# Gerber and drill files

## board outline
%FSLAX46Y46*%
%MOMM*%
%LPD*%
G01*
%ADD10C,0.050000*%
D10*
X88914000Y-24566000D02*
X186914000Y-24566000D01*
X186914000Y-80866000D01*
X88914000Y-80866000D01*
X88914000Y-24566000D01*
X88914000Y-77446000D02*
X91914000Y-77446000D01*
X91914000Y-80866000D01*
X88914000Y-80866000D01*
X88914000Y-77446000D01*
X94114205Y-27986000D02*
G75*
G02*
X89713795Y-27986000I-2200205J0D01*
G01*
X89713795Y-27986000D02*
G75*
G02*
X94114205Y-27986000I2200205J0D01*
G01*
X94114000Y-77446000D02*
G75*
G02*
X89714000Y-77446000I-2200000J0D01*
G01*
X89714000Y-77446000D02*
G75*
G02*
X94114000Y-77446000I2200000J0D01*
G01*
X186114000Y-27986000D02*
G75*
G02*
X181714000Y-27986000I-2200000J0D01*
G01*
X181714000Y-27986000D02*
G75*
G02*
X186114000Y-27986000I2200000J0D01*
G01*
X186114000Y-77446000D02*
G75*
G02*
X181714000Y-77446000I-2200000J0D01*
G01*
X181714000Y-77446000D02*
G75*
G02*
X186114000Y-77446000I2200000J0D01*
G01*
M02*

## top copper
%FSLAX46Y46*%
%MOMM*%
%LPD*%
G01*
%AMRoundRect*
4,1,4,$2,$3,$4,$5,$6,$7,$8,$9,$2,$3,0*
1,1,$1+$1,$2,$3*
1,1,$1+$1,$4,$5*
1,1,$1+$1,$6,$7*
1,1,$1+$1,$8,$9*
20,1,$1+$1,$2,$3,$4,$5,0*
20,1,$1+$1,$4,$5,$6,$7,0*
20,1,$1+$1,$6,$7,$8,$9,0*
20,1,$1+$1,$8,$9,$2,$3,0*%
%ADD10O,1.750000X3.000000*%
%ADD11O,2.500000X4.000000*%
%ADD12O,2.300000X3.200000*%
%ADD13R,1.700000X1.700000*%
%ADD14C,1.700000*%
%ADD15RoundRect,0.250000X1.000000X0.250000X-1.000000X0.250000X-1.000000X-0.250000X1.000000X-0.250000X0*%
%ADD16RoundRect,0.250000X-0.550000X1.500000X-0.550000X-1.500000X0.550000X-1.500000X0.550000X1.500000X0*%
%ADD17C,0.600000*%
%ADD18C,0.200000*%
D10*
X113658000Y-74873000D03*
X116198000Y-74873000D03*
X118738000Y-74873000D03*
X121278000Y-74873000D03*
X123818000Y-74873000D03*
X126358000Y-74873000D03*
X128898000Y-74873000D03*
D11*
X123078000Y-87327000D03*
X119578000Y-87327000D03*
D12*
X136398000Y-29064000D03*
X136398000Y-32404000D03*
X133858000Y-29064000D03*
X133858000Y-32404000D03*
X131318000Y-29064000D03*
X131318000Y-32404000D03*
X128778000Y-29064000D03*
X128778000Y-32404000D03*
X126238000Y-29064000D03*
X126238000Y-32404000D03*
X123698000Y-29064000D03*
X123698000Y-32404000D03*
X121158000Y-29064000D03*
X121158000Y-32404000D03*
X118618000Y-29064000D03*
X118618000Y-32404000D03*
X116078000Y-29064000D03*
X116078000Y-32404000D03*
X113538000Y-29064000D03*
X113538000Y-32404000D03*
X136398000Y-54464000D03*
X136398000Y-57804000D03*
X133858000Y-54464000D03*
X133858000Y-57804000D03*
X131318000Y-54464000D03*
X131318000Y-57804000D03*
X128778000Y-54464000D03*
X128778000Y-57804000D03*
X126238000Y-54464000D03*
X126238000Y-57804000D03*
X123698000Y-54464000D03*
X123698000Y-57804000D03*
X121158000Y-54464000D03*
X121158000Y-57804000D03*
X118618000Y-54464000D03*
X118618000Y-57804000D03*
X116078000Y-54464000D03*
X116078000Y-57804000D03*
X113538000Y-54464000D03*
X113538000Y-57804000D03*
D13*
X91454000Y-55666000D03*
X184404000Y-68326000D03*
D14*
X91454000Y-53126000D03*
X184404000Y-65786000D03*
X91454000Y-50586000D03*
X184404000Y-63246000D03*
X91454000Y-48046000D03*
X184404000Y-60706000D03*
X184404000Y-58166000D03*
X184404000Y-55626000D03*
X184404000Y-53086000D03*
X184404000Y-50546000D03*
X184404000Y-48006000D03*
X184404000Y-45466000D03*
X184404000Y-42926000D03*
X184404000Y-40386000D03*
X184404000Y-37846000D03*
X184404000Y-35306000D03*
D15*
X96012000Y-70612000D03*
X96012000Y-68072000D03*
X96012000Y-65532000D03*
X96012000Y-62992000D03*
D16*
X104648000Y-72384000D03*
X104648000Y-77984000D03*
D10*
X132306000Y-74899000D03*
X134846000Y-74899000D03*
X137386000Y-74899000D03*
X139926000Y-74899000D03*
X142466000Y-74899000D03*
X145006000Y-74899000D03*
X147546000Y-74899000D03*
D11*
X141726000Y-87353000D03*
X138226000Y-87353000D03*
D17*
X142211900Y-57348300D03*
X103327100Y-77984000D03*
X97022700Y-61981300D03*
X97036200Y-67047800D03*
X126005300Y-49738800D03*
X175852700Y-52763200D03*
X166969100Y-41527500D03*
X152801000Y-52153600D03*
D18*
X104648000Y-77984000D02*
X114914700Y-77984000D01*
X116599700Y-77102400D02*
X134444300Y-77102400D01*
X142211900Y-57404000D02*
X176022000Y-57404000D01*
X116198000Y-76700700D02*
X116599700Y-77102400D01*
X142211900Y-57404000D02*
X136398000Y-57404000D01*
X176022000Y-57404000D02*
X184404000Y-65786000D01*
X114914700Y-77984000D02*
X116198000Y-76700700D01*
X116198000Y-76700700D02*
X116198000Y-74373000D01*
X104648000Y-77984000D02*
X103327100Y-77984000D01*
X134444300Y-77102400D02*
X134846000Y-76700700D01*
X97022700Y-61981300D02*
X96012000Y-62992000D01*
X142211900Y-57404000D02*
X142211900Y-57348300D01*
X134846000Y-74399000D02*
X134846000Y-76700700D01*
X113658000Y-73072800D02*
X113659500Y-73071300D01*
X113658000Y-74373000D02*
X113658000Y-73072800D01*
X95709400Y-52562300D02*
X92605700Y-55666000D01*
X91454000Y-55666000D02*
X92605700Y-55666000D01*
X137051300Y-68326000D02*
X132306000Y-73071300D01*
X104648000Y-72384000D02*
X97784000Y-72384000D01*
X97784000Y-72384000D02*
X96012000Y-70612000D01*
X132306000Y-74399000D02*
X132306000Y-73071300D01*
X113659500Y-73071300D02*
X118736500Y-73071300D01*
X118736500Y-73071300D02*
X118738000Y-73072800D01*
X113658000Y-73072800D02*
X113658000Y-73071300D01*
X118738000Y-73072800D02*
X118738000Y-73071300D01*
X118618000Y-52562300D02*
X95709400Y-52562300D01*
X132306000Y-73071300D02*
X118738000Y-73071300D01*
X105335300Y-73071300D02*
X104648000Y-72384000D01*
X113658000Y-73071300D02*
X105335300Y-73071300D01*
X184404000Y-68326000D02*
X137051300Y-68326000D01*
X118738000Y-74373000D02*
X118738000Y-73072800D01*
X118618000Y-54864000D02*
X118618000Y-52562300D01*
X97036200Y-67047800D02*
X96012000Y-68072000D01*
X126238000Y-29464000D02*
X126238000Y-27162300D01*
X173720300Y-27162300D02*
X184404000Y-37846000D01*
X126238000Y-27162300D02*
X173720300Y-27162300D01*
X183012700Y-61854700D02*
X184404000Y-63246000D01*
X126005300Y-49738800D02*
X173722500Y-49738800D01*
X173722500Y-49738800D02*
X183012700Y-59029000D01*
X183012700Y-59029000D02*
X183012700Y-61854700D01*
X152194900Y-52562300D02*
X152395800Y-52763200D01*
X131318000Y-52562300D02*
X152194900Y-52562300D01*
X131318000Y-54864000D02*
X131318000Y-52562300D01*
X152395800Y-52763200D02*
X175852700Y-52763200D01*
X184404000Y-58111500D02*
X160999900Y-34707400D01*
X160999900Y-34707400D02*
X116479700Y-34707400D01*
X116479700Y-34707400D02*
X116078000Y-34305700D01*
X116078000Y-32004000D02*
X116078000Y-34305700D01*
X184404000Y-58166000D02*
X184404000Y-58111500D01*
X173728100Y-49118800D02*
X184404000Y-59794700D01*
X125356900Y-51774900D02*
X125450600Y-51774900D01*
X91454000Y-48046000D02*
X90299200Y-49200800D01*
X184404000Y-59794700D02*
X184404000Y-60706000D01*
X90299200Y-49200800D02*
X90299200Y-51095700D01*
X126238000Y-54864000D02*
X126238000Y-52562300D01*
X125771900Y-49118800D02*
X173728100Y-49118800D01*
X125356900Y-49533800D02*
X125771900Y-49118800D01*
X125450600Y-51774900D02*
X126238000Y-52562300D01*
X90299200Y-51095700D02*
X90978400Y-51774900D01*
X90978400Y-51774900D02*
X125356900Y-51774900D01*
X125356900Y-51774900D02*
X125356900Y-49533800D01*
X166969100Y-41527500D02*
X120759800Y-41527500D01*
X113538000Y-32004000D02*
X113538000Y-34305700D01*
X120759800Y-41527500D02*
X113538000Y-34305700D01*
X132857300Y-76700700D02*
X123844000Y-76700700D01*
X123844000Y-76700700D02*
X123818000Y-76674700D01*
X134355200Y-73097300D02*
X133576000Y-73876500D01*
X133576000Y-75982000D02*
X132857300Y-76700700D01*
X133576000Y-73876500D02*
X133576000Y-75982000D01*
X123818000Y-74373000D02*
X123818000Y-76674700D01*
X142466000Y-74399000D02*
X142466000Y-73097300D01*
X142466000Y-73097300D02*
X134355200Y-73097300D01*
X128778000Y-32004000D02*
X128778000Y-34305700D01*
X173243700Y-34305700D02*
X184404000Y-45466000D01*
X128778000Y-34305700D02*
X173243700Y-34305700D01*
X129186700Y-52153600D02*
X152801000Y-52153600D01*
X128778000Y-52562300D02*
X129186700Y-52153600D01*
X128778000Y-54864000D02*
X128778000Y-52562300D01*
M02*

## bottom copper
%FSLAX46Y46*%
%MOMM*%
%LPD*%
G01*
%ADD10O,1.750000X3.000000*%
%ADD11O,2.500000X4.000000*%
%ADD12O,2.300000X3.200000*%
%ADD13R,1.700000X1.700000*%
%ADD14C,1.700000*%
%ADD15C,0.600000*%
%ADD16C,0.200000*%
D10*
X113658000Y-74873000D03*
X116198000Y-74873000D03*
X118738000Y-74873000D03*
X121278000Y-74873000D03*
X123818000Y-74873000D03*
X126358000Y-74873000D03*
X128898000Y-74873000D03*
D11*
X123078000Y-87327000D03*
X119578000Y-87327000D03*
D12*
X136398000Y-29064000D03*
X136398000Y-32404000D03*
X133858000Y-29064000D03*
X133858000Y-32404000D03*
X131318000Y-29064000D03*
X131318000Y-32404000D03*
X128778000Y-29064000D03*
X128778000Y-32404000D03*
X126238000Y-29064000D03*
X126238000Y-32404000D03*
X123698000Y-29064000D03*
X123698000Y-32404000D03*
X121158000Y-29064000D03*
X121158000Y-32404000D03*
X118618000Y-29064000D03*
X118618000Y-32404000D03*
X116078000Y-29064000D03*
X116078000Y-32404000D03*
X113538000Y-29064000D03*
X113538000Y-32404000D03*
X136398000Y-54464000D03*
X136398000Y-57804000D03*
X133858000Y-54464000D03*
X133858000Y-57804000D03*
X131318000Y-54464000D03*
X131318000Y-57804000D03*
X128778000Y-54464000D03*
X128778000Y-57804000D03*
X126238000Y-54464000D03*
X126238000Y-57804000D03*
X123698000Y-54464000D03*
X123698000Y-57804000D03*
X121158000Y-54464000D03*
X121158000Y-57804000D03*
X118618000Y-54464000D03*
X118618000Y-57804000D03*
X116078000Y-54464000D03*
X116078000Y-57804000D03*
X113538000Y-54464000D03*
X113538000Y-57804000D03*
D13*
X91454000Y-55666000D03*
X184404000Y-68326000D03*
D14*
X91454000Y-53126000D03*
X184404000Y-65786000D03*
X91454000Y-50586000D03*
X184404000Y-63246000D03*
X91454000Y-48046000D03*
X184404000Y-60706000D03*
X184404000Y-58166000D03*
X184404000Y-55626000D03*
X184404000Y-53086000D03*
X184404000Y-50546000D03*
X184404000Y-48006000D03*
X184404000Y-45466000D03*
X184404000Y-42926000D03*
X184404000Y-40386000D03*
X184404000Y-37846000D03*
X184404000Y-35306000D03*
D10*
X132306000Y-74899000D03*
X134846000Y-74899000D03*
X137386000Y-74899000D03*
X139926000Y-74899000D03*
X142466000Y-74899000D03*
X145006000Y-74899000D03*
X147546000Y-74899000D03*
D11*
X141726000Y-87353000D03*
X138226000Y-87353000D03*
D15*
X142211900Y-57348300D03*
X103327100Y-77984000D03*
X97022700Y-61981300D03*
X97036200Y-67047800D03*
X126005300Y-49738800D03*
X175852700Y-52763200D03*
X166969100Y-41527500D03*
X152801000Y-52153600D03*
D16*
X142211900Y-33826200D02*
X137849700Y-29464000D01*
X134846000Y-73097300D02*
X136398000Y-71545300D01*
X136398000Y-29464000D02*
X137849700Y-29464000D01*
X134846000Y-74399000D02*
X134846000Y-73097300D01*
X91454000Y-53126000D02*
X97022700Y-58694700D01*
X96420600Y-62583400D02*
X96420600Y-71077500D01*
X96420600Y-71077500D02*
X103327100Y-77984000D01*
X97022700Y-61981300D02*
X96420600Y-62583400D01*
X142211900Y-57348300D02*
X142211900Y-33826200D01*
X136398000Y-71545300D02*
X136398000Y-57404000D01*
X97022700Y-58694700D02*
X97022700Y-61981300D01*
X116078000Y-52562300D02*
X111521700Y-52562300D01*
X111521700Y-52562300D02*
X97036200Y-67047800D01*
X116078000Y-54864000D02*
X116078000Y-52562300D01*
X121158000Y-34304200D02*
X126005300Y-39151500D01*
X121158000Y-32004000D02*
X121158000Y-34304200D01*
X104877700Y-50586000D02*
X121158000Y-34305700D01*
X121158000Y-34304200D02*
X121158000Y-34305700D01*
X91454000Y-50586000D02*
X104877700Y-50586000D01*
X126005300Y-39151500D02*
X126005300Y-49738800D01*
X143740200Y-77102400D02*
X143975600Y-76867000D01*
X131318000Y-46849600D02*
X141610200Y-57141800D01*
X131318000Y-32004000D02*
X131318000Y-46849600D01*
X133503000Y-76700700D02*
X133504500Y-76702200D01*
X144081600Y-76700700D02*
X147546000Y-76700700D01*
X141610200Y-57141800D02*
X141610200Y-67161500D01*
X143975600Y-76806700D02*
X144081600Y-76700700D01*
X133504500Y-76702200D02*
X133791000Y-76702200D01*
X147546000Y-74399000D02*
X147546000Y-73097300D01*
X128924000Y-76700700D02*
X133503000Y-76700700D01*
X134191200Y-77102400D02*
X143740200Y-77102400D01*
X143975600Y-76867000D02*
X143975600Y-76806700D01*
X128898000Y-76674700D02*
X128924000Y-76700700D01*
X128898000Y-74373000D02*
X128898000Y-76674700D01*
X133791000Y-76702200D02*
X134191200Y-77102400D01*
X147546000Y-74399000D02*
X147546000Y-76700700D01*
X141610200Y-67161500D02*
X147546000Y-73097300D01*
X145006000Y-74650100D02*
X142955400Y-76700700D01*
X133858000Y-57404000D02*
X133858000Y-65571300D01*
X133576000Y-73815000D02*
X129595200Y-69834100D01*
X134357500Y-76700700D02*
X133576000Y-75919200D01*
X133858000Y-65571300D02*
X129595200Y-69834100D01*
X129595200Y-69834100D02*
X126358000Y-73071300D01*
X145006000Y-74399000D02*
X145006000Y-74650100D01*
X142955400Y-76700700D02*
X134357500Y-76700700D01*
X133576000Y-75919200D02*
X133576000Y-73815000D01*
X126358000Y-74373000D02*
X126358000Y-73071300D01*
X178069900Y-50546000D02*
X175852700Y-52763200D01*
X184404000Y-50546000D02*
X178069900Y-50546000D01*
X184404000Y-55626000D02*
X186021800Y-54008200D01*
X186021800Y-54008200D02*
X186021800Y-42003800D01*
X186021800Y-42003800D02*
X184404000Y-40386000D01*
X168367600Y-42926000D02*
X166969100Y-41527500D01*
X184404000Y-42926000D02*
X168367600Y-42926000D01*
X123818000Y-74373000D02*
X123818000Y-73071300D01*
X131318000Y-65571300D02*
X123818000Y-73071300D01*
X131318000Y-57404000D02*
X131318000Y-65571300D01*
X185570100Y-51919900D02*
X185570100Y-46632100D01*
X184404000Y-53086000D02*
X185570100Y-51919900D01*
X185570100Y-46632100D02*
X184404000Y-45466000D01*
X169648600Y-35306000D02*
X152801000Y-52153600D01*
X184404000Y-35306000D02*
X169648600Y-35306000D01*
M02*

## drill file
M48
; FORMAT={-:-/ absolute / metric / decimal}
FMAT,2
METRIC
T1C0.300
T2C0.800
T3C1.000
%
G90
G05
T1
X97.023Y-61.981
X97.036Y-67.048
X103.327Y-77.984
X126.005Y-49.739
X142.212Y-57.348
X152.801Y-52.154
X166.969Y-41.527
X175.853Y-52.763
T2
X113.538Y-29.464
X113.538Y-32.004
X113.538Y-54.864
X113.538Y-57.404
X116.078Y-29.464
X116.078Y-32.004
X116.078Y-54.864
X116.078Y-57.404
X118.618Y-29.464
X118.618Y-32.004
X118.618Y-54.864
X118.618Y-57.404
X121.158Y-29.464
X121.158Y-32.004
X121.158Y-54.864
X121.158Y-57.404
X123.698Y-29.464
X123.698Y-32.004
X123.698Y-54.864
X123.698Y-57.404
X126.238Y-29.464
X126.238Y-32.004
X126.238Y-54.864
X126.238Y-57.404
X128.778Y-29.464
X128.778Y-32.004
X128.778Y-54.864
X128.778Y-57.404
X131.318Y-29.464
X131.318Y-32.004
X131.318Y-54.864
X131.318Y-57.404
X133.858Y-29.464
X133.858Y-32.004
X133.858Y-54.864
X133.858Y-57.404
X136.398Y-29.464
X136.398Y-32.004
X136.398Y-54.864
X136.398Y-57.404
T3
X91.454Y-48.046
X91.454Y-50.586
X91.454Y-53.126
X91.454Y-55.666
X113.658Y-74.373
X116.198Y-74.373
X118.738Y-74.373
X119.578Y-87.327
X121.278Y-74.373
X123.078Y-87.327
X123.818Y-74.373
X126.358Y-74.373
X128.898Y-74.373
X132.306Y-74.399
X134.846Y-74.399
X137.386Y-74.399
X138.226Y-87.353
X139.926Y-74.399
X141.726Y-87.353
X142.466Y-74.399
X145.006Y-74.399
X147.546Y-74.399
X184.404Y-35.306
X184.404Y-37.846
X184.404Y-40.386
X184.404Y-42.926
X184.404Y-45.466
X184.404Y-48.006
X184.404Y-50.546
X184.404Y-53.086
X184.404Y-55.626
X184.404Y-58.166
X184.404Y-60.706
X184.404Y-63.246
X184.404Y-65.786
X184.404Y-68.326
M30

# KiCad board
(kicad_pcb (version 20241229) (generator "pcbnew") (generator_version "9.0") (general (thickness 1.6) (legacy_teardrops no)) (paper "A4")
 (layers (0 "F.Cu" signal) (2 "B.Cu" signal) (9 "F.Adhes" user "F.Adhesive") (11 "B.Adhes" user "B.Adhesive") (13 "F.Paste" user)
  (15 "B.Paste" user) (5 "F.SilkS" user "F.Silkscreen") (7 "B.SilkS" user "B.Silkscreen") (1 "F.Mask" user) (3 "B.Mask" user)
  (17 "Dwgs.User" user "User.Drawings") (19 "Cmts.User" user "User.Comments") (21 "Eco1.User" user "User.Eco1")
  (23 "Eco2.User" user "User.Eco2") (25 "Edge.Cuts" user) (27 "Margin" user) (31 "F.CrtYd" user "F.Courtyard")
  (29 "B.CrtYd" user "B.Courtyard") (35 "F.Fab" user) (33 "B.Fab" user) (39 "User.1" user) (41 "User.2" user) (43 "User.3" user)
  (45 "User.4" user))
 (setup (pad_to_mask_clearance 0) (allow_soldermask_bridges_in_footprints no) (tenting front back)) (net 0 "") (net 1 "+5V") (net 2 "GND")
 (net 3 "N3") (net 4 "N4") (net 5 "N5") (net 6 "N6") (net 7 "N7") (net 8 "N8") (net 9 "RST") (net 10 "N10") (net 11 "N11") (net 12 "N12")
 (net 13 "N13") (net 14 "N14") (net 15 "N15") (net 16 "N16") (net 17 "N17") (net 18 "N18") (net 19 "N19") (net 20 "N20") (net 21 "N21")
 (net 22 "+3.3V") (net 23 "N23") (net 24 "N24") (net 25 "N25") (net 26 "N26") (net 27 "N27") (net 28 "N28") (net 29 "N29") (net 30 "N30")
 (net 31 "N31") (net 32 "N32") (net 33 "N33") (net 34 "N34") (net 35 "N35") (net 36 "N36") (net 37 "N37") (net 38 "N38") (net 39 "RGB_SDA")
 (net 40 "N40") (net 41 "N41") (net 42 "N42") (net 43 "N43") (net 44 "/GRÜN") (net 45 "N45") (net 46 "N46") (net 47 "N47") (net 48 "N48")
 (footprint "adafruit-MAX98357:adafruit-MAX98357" (layer "F.Cu") (at 121.158 81.28 180)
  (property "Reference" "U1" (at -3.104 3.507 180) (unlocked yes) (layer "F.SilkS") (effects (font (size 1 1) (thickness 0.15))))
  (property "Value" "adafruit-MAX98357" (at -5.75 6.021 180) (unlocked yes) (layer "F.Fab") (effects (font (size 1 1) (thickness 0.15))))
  (pad "1" thru_hole oval (at 7.5 6.907 90) (size 3 1.75) (drill 1 (offset -0.5 0)) (layers "*.Cu" "*.Mask") (remove_unused_layers no)
   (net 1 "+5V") (solder_mask_margin 0.0508))
  (pad "2" thru_hole oval (at 4.96 6.907 90) (size 3 1.75) (drill 1 (offset -0.5 0)) (layers "*.Cu" "*.Mask") (remove_unused_layers no)
   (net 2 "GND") (solder_mask_margin 0.0508))
  (pad "3" thru_hole oval (at 2.42 6.907 90) (size 3 1.75) (drill 1 (offset -0.5 0)) (layers "*.Cu" "*.Mask") (remove_unused_layers no)
   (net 1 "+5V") (solder_mask_margin 0.0508))
  (pad "4" thru_hole oval (at -0.12 6.907 90) (size 3 1.75) (drill 1 (offset -0.5 0)) (layers "*.Cu" "*.Mask") (remove_unused_layers no)
   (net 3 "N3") (solder_mask_margin 0.0508))
  (pad "5" thru_hole oval (at -2.66 6.907 90) (size 3 1.75) (drill 1 (offset -0.5 0)) (layers "*.Cu" "*.Mask") (remove_unused_layers no)
   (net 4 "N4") (solder_mask_margin 0.0508))
  (pad "6" thru_hole oval (at -5.2 6.907 90) (size 3 1.75) (drill 1 (offset -0.5 0)) (layers "*.Cu" "*.Mask") (remove_unused_layers no)
   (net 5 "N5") (solder_mask_margin 0.0508))
  (pad "7" thru_hole oval (at -7.74 6.907 90) (size 3 1.75) (drill 1 (offset -0.5 0)) (layers "*.Cu" "*.Mask") (remove_unused_layers no)
   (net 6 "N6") (solder_mask_margin 0.0508))
  (pad "8" thru_hole oval (at -1.92 -6.047) (size 2.5 4) (drill 1) (layers "*.Cu" "*.Mask") (remove_unused_layers no) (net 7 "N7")
   (solder_mask_margin 0.0508))
  (pad "9" thru_hole oval (at 1.58 -6.047) (size 2.5 4) (drill 1) (layers "*.Cu" "*.Mask") (remove_unused_layers no) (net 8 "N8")
   (solder_mask_margin 0.0508)))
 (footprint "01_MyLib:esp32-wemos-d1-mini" (layer "F.Cu") (at 124.968 43.434 -90)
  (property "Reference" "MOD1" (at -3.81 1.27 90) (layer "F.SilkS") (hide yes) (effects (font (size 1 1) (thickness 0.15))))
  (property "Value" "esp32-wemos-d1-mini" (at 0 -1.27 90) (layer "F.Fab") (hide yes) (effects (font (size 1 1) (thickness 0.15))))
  (pad "1" thru_hole oval (at -13.97 -11.43 180) (size 2.3 3.2) (drill 0.8 (offset 0 0.4)) (layers "*.Cu" "*.Mask")
   (remove_unused_layers no) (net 2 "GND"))
  (pad "2" thru_hole oval (at -11.43 -11.43 180) (size 2.3 3.2) (drill 0.8 (offset 0 -0.4)) (layers "*.Cu" "*.Mask")
   (remove_unused_layers no) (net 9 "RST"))
  (pad "3" thru_hole oval (at -13.97 -8.89 180) (size 2.3 3.2) (drill 0.8 (offset 0 0.4)) (layers "*.Cu" "*.Mask") (remove_unused_layers no)
   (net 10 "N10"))
  (pad "4" thru_hole oval (at -11.43 -8.89 180) (size 2.3 3.2) (drill 0.8 (offset 0 -0.4)) (layers "*.Cu" "*.Mask")
   (remove_unused_layers no) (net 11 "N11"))
  (pad "5" thru_hole oval (at -13.97 -6.35 180) (size 2.3 3.2) (drill 0.8 (offset 0 0.4)) (layers "*.Cu" "*.Mask") (remove_unused_layers no)
   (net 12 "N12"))
  (pad "6" thru_hole oval (at -11.43 -6.35 180) (size 2.3 3.2) (drill 0.8 (offset 0 -0.4)) (layers "*.Cu" "*.Mask")
   (remove_unused_layers no) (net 6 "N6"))
  (pad "7" thru_hole oval (at -13.97 -3.81 180) (size 2.3 3.2) (drill 0.8 (offset 0 0.4)) (layers "*.Cu" "*.Mask") (remove_unused_layers no)
   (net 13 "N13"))
  (pad "8" thru_hole oval (at -11.43 -3.81 180) (size 2.3 3.2) (drill 0.8 (offset 0 -0.4)) (layers "*.Cu" "*.Mask")
   (remove_unused_layers no) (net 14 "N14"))
  (pad "9" thru_hole oval (at -13.97 -1.27 180) (size 2.3 3.2) (drill 0.8 (offset 0 0.4)) (layers "*.Cu" "*.Mask") (remove_unused_layers no)
   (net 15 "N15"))
  (pad "10" thru_hole oval (at -11.43 -1.27 180) (size 2.3 3.2) (drill 0.8 (offset 0 -0.4)) (layers "*.Cu" "*.Mask")
   (remove_unused_layers no) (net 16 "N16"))
  (pad "11" thru_hole oval (at -13.97 1.27 180) (size 2.3 3.2) (drill 0.8 (offset 0 0.4)) (layers "*.Cu" "*.Mask") (remove_unused_layers no)
   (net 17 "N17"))
  (pad "12" thru_hole oval (at -11.43 1.27 180) (size 2.3 3.2) (drill 0.8 (offset 0 -0.4)) (layers "*.Cu" "*.Mask")
   (remove_unused_layers no) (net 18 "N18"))
  (pad "13" thru_hole oval (at -13.97 3.81 180) (size 2.3 3.2) (drill 0.8 (offset 0 0.4)) (layers "*.Cu" "*.Mask") (remove_unused_layers no)
   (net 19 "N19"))
  (pad "14" thru_hole oval (at -11.43 3.81 180) (size 2.3 3.2) (drill 0.8 (offset 0 -0.4)) (layers "*.Cu" "*.Mask")
   (remove_unused_layers no) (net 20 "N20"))
  (pad "15" thru_hole oval (at -13.97 6.35 180) (size 2.3 3.2) (drill 0.8 (offset 0 0.4)) (layers "*.Cu" "*.Mask") (remove_unused_layers no)
   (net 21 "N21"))
  (pad "16" thru_hole oval (at -11.43 6.35 180) (size 2.3 3.2) (drill 0.8 (offset 0 -0.4)) (layers "*.Cu" "*.Mask")
   (remove_unused_layers no) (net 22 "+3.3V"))
  (pad "17" thru_hole oval (at -13.97 8.89 180) (size 2.3 3.2) (drill 0.8 (offset 0 0.4)) (layers "*.Cu" "*.Mask") (remove_unused_layers no)
   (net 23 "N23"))
  (pad "18" thru_hole oval (at -11.43 8.89 180) (size 2.3 3.2) (drill 0.8 (offset 0 -0.4)) (layers "*.Cu" "*.Mask")
   (remove_unused_layers no) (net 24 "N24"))
  (pad "19" thru_hole oval (at -13.97 11.43 180) (size 2.3 3.2) (drill 0.8 (offset 0 0.4)) (layers "*.Cu" "*.Mask")
   (remove_unused_layers no) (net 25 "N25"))
  (pad "20" thru_hole oval (at -11.43 11.43 180) (size 2.3 3.2) (drill 0.8 (offset 0 -0.4)) (layers "*.Cu" "*.Mask")
   (remove_unused_layers no) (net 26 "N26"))
  (pad "21" thru_hole oval (at 11.43 -11.43 180) (size 2.3 3.2) (drill 0.8 (offset 0 0.4)) (layers "*.Cu" "*.Mask")
   (remove_unused_layers no) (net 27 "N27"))
  (pad "22" thru_hole oval (at 13.97 -11.43 180) (size 2.3 3.2) (drill 0.8 (offset 0 -0.4)) (layers "*.Cu" "*.Mask")
   (remove_unused_layers no) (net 2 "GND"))
  (pad "23" thru_hole oval (at 11.43 -8.89 180) (size 2.3 3.2) (drill 0.8 (offset 0 0.4)) (layers "*.Cu" "*.Mask") (remove_unused_layers no)
   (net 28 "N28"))
  (pad "24" thru_hole oval (at 13.97 -8.89 180) (size 2.3 3.2) (drill 0.8 (offset 0 -0.4)) (layers "*.Cu" "*.Mask")
   (remove_unused_layers no) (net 5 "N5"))
  (pad "25" thru_hole oval (at 11.43 -6.35 180) (size 2.3 3.2) (drill 0.8 (offset 0 0.4)) (layers "*.Cu" "*.Mask") (remove_unused_layers no)
   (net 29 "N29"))
  (pad "26" thru_hole oval (at 13.97 -6.35 180) (size 2.3 3.2) (drill 0.8 (offset 0 -0.4)) (layers "*.Cu" "*.Mask")
   (remove_unused_layers no) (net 4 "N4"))
  (pad "27" thru_hole oval (at 11.43 -3.81 180) (size 2.3 3.2) (drill 0.8 (offset 0 0.4)) (layers "*.Cu" "*.Mask") (remove_unused_layers no)
   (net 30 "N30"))
  (pad "28" thru_hole oval (at 13.97 -3.81 180) (size 2.3 3.2) (drill 0.8 (offset 0 -0.4)) (layers "*.Cu" "*.Mask")
   (remove_unused_layers no) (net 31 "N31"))
  (pad "29" thru_hole oval (at 11.43 -1.27 180) (size 2.3 3.2) (drill 0.8 (offset 0 0.4)) (layers "*.Cu" "*.Mask") (remove_unused_layers no)
   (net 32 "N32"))
  (pad "30" thru_hole oval (at 13.97 -1.27 180) (size 2.3 3.2) (drill 0.8 (offset 0 -0.4)) (layers "*.Cu" "*.Mask")
   (remove_unused_layers no) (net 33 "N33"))
  (pad "31" thru_hole oval (at 11.43 1.27 180) (size 2.3 3.2) (drill 0.8 (offset 0 0.4)) (layers "*.Cu" "*.Mask") (remove_unused_layers no)
   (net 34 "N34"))
  (pad "32" thru_hole oval (at 13.97 1.27 180) (size 2.3 3.2) (drill 0.8 (offset 0 -0.4)) (layers "*.Cu" "*.Mask") (remove_unused_layers no)
   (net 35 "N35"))
  (pad "33" thru_hole oval (at 11.43 3.81 180) (size 2.3 3.2) (drill 0.8 (offset 0 0.4)) (layers "*.Cu" "*.Mask") (remove_unused_layers no)
   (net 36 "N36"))
  (pad "34" thru_hole oval (at 13.97 3.81 180) (size 2.3 3.2) (drill 0.8 (offset 0 -0.4)) (layers "*.Cu" "*.Mask") (remove_unused_layers no)
   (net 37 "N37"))
  (pad "35" thru_hole oval (at 11.43 6.35 180) (size 2.3 3.2) (drill 0.8 (offset 0 0.4)) (layers "*.Cu" "*.Mask") (remove_unused_layers no)
   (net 1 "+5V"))
  (pad "36" thru_hole oval (at 13.97 6.35 180) (size 2.3 3.2) (drill 0.8 (offset 0 -0.4)) (layers "*.Cu" "*.Mask") (remove_unused_layers no)
   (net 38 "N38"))
  (pad "37" thru_hole oval (at 11.43 8.89 180) (size 2.3 3.2) (drill 0.8 (offset 0 0.4)) (layers "*.Cu" "*.Mask") (remove_unused_layers no)
   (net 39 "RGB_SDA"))
  (pad "38" thru_hole oval (at 13.97 8.89 180) (size 2.3 3.2) (drill 0.8 (offset 0 -0.4)) (layers "*.Cu" "*.Mask") (remove_unused_layers no)
   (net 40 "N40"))
  (pad "39" thru_hole oval (at 11.43 11.43 180) (size 2.3 3.2) (drill 0.8 (offset 0 0.4)) (layers "*.Cu" "*.Mask") (remove_unused_layers no)
   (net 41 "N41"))
  (pad "40" thru_hole oval (at 13.97 11.43 180) (size 2.3 3.2) (drill 0.8 (offset 0 -0.4)) (layers "*.Cu" "*.Mask")
   (remove_unused_layers no) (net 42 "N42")))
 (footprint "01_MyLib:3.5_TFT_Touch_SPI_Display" (layer "F.Cu") (at 88.914 80.866)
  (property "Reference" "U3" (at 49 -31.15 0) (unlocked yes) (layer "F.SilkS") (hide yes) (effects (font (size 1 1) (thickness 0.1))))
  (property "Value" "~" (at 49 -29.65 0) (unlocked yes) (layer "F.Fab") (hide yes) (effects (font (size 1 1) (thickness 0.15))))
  (fp_rect (start 0 -56.3) (end 98 0) (stroke (width 0.05) (type default)) (fill no) (layer "Edge.Cuts"))
  (fp_rect (start 0 -3.42) (end 3 0) (stroke (width 0.05) (type default)) (fill no) (layer "Edge.Cuts"))
  (fp_circle (center 3 -52.88) (end 5.2 -52.91) (stroke (width 0.05) (type default)) (fill no) (layer "Edge.Cuts"))
  (fp_circle (center 3 -3.42) (end 5.2 -3.42) (stroke (width 0.05) (type default)) (fill no) (layer "Edge.Cuts"))
  (fp_circle (center 95 -52.88) (end 92.8 -52.88) (stroke (width 0.05) (type default)) (fill no) (layer "Edge.Cuts"))
  (fp_circle (center 95 -3.42) (end 92.8 -3.42) (stroke (width 0.05) (type default)) (fill no) (layer "Edge.Cuts"))
  (pad "1" thru_hole rect (at 2.54 -25.2 180) (size 1.7 1.7) (drill 1) (layers "*.Cu" "*.Mask") (remove_unused_layers no) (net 1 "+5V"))
  (pad "1" thru_hole rect (at 95.49 -12.54 180) (size 1.7 1.7) (drill 1) (layers "*.Cu" "*.Mask") (remove_unused_layers no) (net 1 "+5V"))
  (pad "2" thru_hole circle (at 2.54 -27.74 180) (size 1.7 1.7) (drill 1) (layers "*.Cu" "*.Mask") (remove_unused_layers no) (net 2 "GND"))
  (pad "2" thru_hole circle (at 95.49 -15.08 180) (size 1.7 1.7) (drill 1) (layers "*.Cu" "*.Mask") (remove_unused_layers no) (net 2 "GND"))
  (pad "3" thru_hole circle (at 2.54 -30.28 180) (size 1.7 1.7) (drill 1) (layers "*.Cu" "*.Mask") (remove_unused_layers no) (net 20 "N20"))
  (pad "3" thru_hole circle (at 95.49 -17.62 180) (size 1.7 1.7) (drill 1) (layers "*.Cu" "*.Mask") (remove_unused_layers no) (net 20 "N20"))
  (pad "4" thru_hole circle (at 2.54 -32.82 180) (size 1.7 1.7) (drill 1) (layers "*.Cu" "*.Mask") (remove_unused_layers no) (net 32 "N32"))
  (pad "4" thru_hole circle (at 95.49 -20.16 180) (size 1.7 1.7) (drill 1) (layers "*.Cu" "*.Mask") (remove_unused_layers no) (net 32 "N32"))
  (pad "5" thru_hole circle (at 95.49 -22.7 180) (size 1.7 1.7) (drill 1) (layers "*.Cu" "*.Mask") (remove_unused_layers no) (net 24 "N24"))
  (pad "6" thru_hole circle (at 95.49 -25.24 180) (size 1.7 1.7) (drill 1) (layers "*.Cu" "*.Mask") (remove_unused_layers no) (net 17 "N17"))
  (pad "7" thru_hole circle (at 95.49 -27.78 180) (size 1.7 1.7) (drill 1) (layers "*.Cu" "*.Mask") (remove_unused_layers no) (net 14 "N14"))
  (pad "8" thru_hole circle (at 95.49 -30.32 180) (size 1.7 1.7) (drill 1) (layers "*.Cu" "*.Mask") (remove_unused_layers no) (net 29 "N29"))
  (pad "9" thru_hole circle (at 95.49 -32.86 180) (size 1.7 1.7) (drill 1) (layers "*.Cu" "*.Mask") (remove_unused_layers no) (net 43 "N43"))
  (pad "10" thru_hole circle (at 95.49 -35.4 180) (size 1.7 1.7) (drill 1) (layers "*.Cu" "*.Mask") (remove_unused_layers no) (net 14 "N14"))
  (pad "11" thru_hole circle (at 95.49 -37.94 180) (size 1.7 1.7) (drill 1) (layers "*.Cu" "*.Mask") (remove_unused_layers no)
   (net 26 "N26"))
  (pad "12" thru_hole circle (at 95.49 -40.48 180) (size 1.7 1.7) (drill 1) (layers "*.Cu" "*.Mask") (remove_unused_layers no)
   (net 17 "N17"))
  (pad "13" thru_hole circle (at 95.49 -43.02 180) (size 1.7 1.7) (drill 1) (layers "*.Cu" "*.Mask") (remove_unused_layers no)
   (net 15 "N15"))
  (pad "14" thru_hole circle (at 95.49 -45.56 180) (size 1.7 1.7) (drill 1) (layers "*.Cu" "*.Mask") (remove_unused_layers no)
   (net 30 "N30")))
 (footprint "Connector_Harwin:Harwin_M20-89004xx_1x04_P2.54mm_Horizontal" (layer "F.Cu") (at 90.487 66.802 180)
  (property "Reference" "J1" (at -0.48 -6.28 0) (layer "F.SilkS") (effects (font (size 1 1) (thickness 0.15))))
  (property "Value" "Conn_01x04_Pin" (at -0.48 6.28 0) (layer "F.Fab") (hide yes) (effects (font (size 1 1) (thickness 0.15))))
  (pad "1" smd roundrect (at -5.525 -3.81 180) (size 2.5 1) (layers "F.Cu" "F.Mask" "F.Paste") (roundrect_rratio 0.25) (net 1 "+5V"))
  (pad "2" smd roundrect (at -5.525 -1.27 180) (size 2.5 1) (layers "F.Cu" "F.Mask" "F.Paste") (roundrect_rratio 0.25) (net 39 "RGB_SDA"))
  (pad "3" smd roundrect (at -5.525 1.27 180) (size 2.5 1) (layers "F.Cu" "F.Mask" "F.Paste") (roundrect_rratio 0.25) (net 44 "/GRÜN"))
  (pad "4" smd roundrect (at -5.525 3.81 180) (size 2.5 1) (layers "F.Cu" "F.Mask" "F.Paste") (roundrect_rratio 0.25) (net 2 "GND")))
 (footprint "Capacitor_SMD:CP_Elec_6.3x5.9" (layer "F.Cu") (at 104.648 75.184 -90)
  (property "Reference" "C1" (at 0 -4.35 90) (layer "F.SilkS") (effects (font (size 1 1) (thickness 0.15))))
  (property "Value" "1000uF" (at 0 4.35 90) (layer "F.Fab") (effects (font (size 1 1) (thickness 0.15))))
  (pad "1" smd roundrect (at -2.8 0 270) (size 3.5 1.6) (layers "F.Cu" "F.Mask" "F.Paste") (roundrect_rratio 0.15625) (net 1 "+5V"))
  (pad "2" smd roundrect (at 2.8 0 270) (size 3.5 1.6) (layers "F.Cu" "F.Mask" "F.Paste") (roundrect_rratio 0.15625) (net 2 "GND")))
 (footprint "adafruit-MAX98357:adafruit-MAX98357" (layer "F.Cu") (at 139.806 81.306 180)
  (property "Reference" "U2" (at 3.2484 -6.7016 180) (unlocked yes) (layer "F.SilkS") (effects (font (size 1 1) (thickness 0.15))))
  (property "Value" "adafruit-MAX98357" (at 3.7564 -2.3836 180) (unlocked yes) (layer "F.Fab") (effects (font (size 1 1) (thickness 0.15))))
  (pad "1" thru_hole oval (at 7.5 6.907 90) (size 3 1.75) (drill 1 (offset -0.5 0)) (layers "*.Cu" "*.Mask") (remove_unused_layers no)
   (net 1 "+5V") (solder_mask_margin 0.0508))
  (pad "2" thru_hole oval (at 4.96 6.907 90) (size 3 1.75) (drill 1 (offset -0.5 0)) (layers "*.Cu" "*.Mask") (remove_unused_layers no)
   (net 2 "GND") (solder_mask_margin 0.0508))
  (pad "3" thru_hole oval (at 2.42 6.907 90) (size 3 1.75) (drill 1 (offset -0.5 0)) (layers "*.Cu" "*.Mask") (remove_unused_layers no)
   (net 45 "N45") (solder_mask_margin 0.0508))
  (pad "4" thru_hole oval (at -0.12 6.907 90) (size 3 1.75) (drill 1 (offset -0.5 0)) (layers "*.Cu" "*.Mask") (remove_unused_layers no)
   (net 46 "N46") (solder_mask_margin 0.0508))
  (pad "5" thru_hole oval (at -2.66 6.907 90) (size 3 1.75) (drill 1 (offset -0.5 0)) (layers "*.Cu" "*.Mask") (remove_unused_layers no)
   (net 4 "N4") (solder_mask_margin 0.0508))
  (pad "6" thru_hole oval (at -5.2 6.907 90) (size 3 1.75) (drill 1 (offset -0.5 0)) (layers "*.Cu" "*.Mask") (remove_unused_layers no)
   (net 5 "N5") (solder_mask_margin 0.0508))
  (pad "7" thru_hole oval (at -7.74 6.907 90) (size 3 1.75) (drill 1 (offset -0.5 0)) (layers "*.Cu" "*.Mask") (remove_unused_layers no)
   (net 6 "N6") (solder_mask_margin 0.0508))
  (pad "8" thru_hole oval (at -1.92 -6.047) (size 2.5 4) (drill 1) (layers "*.Cu" "*.Mask") (remove_unused_layers no) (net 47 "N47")
   (solder_mask_margin 0.0508))
  (pad "9" thru_hole oval (at 1.58 -6.047) (size 2.5 4) (drill 1) (layers "*.Cu" "*.Mask") (remove_unused_layers no) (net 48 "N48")
   (solder_mask_margin 0.0508)))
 (segment (start 104.648 77.984) (end 114.9147 77.984) (width 0.2) (layer "F.Cu") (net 2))
 (segment (start 116.5997 77.1024) (end 134.4443 77.1024) (width 0.2) (layer "F.Cu") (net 2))
 (segment (start 142.2119 57.404) (end 176.022 57.404) (width 0.2) (layer "F.Cu") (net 2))
 (segment (start 116.198 76.7007) (end 116.5997 77.1024) (width 0.2) (layer "F.Cu") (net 2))
 (segment (start 142.2119 57.404) (end 136.398 57.404) (width 0.2) (layer "F.Cu") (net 2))
 (segment (start 176.022 57.404) (end 184.404 65.786) (width 0.2) (layer "F.Cu") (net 2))
 (segment (start 114.9147 77.984) (end 116.198 76.7007) (width 0.2) (layer "F.Cu") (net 2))
 (segment (start 116.198 76.7007) (end 116.198 74.373) (width 0.2) (layer "F.Cu") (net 2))
 (segment (start 104.648 77.984) (end 103.3271 77.984) (width 0.2) (layer "F.Cu") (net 2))
 (segment (start 134.4443 77.1024) (end 134.846 76.7007) (width 0.2) (layer "F.Cu") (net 2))
 (segment (start 97.0227 61.9813) (end 96.012 62.992) (width 0.2) (layer "F.Cu") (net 2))
 (segment (start 142.2119 57.404) (end 142.2119 57.3483) (width 0.2) (layer "F.Cu") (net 2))
 (segment (start 134.846 74.399) (end 134.846 76.7007) (width 0.2) (layer "F.Cu") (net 2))
 (via (at 142.2119 57.3483) (size 0.6) (drill 0.3) (layers "F.Cu" "B.Cu") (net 2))
 (via (at 103.3271 77.984) (size 0.6) (drill 0.3) (layers "F.Cu" "B.Cu") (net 2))
 (via (at 97.0227 61.9813) (size 0.6) (drill 0.3) (layers "F.Cu" "B.Cu") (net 2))
 (segment (start 142.2119 33.8262) (end 137.8497 29.464) (width 0.2) (layer "B.Cu") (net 2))
 (segment (start 134.846 73.0973) (end 136.398 71.5453) (width 0.2) (layer "B.Cu") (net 2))
 (segment (start 136.398 29.464) (end 137.8497 29.464) (width 0.2) (layer "B.Cu") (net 2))
 (segment (start 134.846 74.399) (end 134.846 73.0973) (width 0.2) (layer "B.Cu") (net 2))
 (segment (start 91.454 53.126) (end 97.0227 58.6947) (width 0.2) (layer "B.Cu") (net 2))
 (segment (start 96.4206 62.5834) (end 96.4206 71.0775) (width 0.2) (layer "B.Cu") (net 2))
 (segment (start 96.4206 71.0775) (end 103.3271 77.984) (width 0.2) (layer "B.Cu") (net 2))
 (segment (start 97.0227 61.9813) (end 96.4206 62.5834) (width 0.2) (layer "B.Cu") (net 2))
 (segment (start 142.2119 57.3483) (end 142.2119 33.8262) (width 0.2) (layer "B.Cu") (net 2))
 (segment (start 136.398 71.5453) (end 136.398 57.404) (width 0.2) (layer "B.Cu") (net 2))
 (segment (start 97.0227 58.6947) (end 97.0227 61.9813) (width 0.2) (layer "B.Cu") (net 2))
 (segment (start 113.658 73.0728) (end 113.6595 73.0713) (width 0.2) (layer "F.Cu") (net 1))
 (segment (start 113.658 74.373) (end 113.658 73.0728) (width 0.2) (layer "F.Cu") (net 1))
 (segment (start 95.7094 52.5623) (end 92.6057 55.666) (width 0.2) (layer "F.Cu") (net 1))
 (segment (start 91.454 55.666) (end 92.6057 55.666) (width 0.2) (layer "F.Cu") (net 1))
 (segment (start 137.0513 68.326) (end 132.306 73.0713) (width 0.2) (layer "F.Cu") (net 1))
 (segment (start 104.648 72.384) (end 97.784 72.384) (width 0.2) (layer "F.Cu") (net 1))
 (segment (start 97.784 72.384) (end 96.012 70.612) (width 0.2) (layer "F.Cu") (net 1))
 (segment (start 132.306 74.399) (end 132.306 73.0713) (width 0.2) (layer "F.Cu") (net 1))
 (segment (start 113.6595 73.0713) (end 118.7365 73.0713) (width 0.2) (layer "F.Cu") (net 1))
 (segment (start 118.7365 73.0713) (end 118.738 73.0728) (width 0.2) (layer "F.Cu") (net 1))
 (segment (start 113.658 73.0728) (end 113.658 73.0713) (width 0.2) (layer "F.Cu") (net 1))
 (segment (start 118.738 73.0728) (end 118.738 73.0713) (width 0.2) (layer "F.Cu") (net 1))
 (segment (start 118.618 52.5623) (end 95.7094 52.5623) (width 0.2) (layer "F.Cu") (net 1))
 (segment (start 132.306 73.0713) (end 118.738 73.0713) (width 0.2) (layer "F.Cu") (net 1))
 (segment (start 105.3353 73.0713) (end 104.648 72.384) (width 0.2) (layer "F.Cu") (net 1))
 (segment (start 113.658 73.0713) (end 105.3353 73.0713) (width 0.2) (layer "F.Cu") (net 1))
 (segment (start 184.404 68.326) (end 137.0513 68.326) (width 0.2) (layer "F.Cu") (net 1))
 (segment (start 118.738 74.373) (end 118.738 73.0728) (width 0.2) (layer "F.Cu") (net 1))
 (segment (start 118.618 54.864) (end 118.618 52.5623) (width 0.2) (layer "F.Cu") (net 1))
 (segment (start 97.0362 67.0478) (end 96.012 68.072) (width 0.2) (layer "F.Cu") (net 39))
 (via (at 97.0362 67.0478) (size 0.6) (drill 0.3) (layers "F.Cu" "B.Cu") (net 39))
 (segment (start 116.078 52.5623) (end 111.5217 52.5623) (width 0.2) (layer "B.Cu") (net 39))
 (segment (start 111.5217 52.5623) (end 97.0362 67.0478) (width 0.2) (layer "B.Cu") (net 39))
 (segment (start 116.078 54.864) (end 116.078 52.5623) (width 0.2) (layer "B.Cu") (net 39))
 (segment (start 126.238 29.464) (end 126.238 27.1623) (width 0.2) (layer "F.Cu") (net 15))
 (segment (start 173.7203 27.1623) (end 184.404 37.846) (width 0.2) (layer "F.Cu") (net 15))
 (segment (start 126.238 27.1623) (end 173.7203 27.1623) (width 0.2) (layer "F.Cu") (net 15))
 (segment (start 183.0127 61.8547) (end 184.404 63.246) (width 0.2) (layer "F.Cu") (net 20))
 (segment (start 126.0053 49.7388) (end 173.7225 49.7388) (width 0.2) (layer "F.Cu") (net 20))
 (segment (start 173.7225 49.7388) (end 183.0127 59.029) (width 0.2) (layer "F.Cu") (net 20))
 (segment (start 183.0127 59.029) (end 183.0127 61.8547) (width 0.2) (layer "F.Cu") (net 20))
 (via (at 126.0053 49.7388) (size 0.6) (drill 0.3) (layers "F.Cu" "B.Cu") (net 20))
 (segment (start 121.158 34.3042) (end 126.0053 39.1515) (width 0.2) (layer "B.Cu") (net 20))
 (segment (start 121.158 32.004) (end 121.158 34.3042) (width 0.2) (layer "B.Cu") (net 20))
 (segment (start 104.8777 50.586) (end 121.158 34.3057) (width 0.2) (layer "B.Cu") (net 20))
 (segment (start 121.158 34.3042) (end 121.158 34.3057) (width 0.2) (layer "B.Cu") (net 20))
 (segment (start 91.454 50.586) (end 104.8777 50.586) (width 0.2) (layer "B.Cu") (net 20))
 (segment (start 126.0053 39.1515) (end 126.0053 49.7388) (width 0.2) (layer "B.Cu") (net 20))
 (segment (start 143.7402 77.1024) (end 143.9756 76.867) (width 0.2) (layer "B.Cu") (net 6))
 (segment (start 131.318 46.8496) (end 141.6102 57.1418) (width 0.2) (layer "B.Cu") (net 6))
 (segment (start 131.318 32.004) (end 131.318 46.8496) (width 0.2) (layer "B.Cu") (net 6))
 (segment (start 133.503 76.7007) (end 133.5045 76.7022) (width 0.2) (layer "B.Cu") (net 6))
 (segment (start 144.0816 76.7007) (end 147.546 76.7007) (width 0.2) (layer "B.Cu") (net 6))
 (segment (start 141.6102 57.1418) (end 141.6102 67.1615) (width 0.2) (layer "B.Cu") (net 6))
 (segment (start 143.9756 76.8067) (end 144.0816 76.7007) (width 0.2) (layer "B.Cu") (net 6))
 (segment (start 133.5045 76.7022) (end 133.791 76.7022) (width 0.2) (layer "B.Cu") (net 6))
 (segment (start 147.546 74.399) (end 147.546 73.0973) (width 0.2) (layer "B.Cu") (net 6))
 (segment (start 128.924 76.7007) (end 133.503 76.7007) (width 0.2) (layer "B.Cu") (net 6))
 (segment (start 134.1912 77.1024) (end 143.7402 77.1024) (width 0.2) (layer "B.Cu") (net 6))
 (segment (start 143.9756 76.867) (end 143.9756 76.8067) (width 0.2) (layer "B.Cu") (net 6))
 (segment (start 128.898 76.6747) (end 128.924 76.7007) (width 0.2) (layer "B.Cu") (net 6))
 (segment (start 128.898 74.373) (end 128.898 76.6747) (width 0.2) (layer "B.Cu") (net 6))
 (segment (start 133.791 76.7022) (end 134.1912 77.1024) (width 0.2) (layer "B.Cu") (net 6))
 (segment (start 147.546 74.399) (end 147.546 76.7007) (width 0.2) (layer "B.Cu") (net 6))
 (segment (start 141.6102 67.1615) (end 147.546 73.0973) (width 0.2) (layer "B.Cu") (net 6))
 (segment (start 145.006 74.6501) (end 142.9554 76.7007) (width 0.2) (layer "B.Cu") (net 5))
 (segment (start 133.858 57.404) (end 133.858 65.5713) (width 0.2) (layer "B.Cu") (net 5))
 (segment (start 133.576 73.815) (end 129.5952 69.8341) (width 0.2) (layer "B.Cu") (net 5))
 (segment (start 134.3575 76.7007) (end 133.576 75.9192) (width 0.2) (layer "B.Cu") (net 5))
 (segment (start 133.858 65.5713) (end 129.5952 69.8341) (width 0.2) (layer "B.Cu") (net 5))
 (segment (start 129.5952 69.8341) (end 126.358 73.0713) (width 0.2) (layer "B.Cu") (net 5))
 (segment (start 145.006 74.399) (end 145.006 74.6501) (width 0.2) (layer "B.Cu") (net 5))
 (segment (start 142.9554 76.7007) (end 134.3575 76.7007) (width 0.2) (layer "B.Cu") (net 5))
 (segment (start 133.576 75.9192) (end 133.576 73.815) (width 0.2) (layer "B.Cu") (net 5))
 (segment (start 126.358 74.373) (end 126.358 73.0713) (width 0.2) (layer "B.Cu") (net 5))
 (segment (start 152.1949 52.5623) (end 152.3958 52.7632) (width 0.2) (layer "F.Cu") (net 29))
 (segment (start 131.318 52.5623) (end 152.1949 52.5623) (width 0.2) (layer "F.Cu") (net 29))
 (segment (start 131.318 54.864) (end 131.318 52.5623) (width 0.2) (layer "F.Cu") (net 29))
 (segment (start 152.3958 52.7632) (end 175.8527 52.7632) (width 0.2) (layer "F.Cu") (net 29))
 (via (at 175.8527 52.7632) (size 0.6) (drill 0.3) (layers "F.Cu" "B.Cu") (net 29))
 (segment (start 178.0699 50.546) (end 175.8527 52.7632) (width 0.2) (layer "B.Cu") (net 29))
 (segment (start 184.404 50.546) (end 178.0699 50.546) (width 0.2) (layer "B.Cu") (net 29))
 (segment (start 184.404 58.1115) (end 160.9999 34.7074) (width 0.2) (layer "F.Cu") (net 24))
 (segment (start 160.9999 34.7074) (end 116.4797 34.7074) (width 0.2) (layer "F.Cu") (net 24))
 (segment (start 116.4797 34.7074) (end 116.078 34.3057) (width 0.2) (layer "F.Cu") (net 24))
 (segment (start 116.078 32.004) (end 116.078 34.3057) (width 0.2) (layer "F.Cu") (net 24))
 (segment (start 184.404 58.166) (end 184.404 58.1115) (width 0.2) (layer "F.Cu") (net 24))
 (segment (start 173.7281 49.1188) (end 184.404 59.7947) (width 0.2) (layer "F.Cu") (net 32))
 (segment (start 125.3569 51.7749) (end 125.4506 51.7749) (width 0.2) (layer "F.Cu") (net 32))
 (segment (start 91.454 48.046) (end 90.2992 49.2008) (width 0.2) (layer "F.Cu") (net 32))
 (segment (start 184.404 59.7947) (end 184.404 60.706) (width 0.2) (layer "F.Cu") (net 32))
 (segment (start 90.2992 49.2008) (end 90.2992 51.0957) (width 0.2) (layer "F.Cu") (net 32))
 (segment (start 126.238 54.864) (end 126.238 52.5623) (width 0.2) (layer "F.Cu") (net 32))
 (segment (start 125.7719 49.1188) (end 173.7281 49.1188) (width 0.2) (layer "F.Cu") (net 32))
 (segment (start 125.3569 49.5338) (end 125.7719 49.1188) (width 0.2) (layer "F.Cu") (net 32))
 (segment (start 125.4506 51.7749) (end 126.238 52.5623) (width 0.2) (layer "F.Cu") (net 32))
 (segment (start 90.2992 51.0957) (end 90.9784 51.7749) (width 0.2) (layer "F.Cu") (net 32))
 (segment (start 90.9784 51.7749) (end 125.3569 51.7749) (width 0.2) (layer "F.Cu") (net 32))
 (segment (start 125.3569 51.7749) (end 125.3569 49.5338) (width 0.2) (layer "F.Cu") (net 32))
 (segment (start 184.404 55.626) (end 186.0218 54.0082) (width 0.2) (layer "B.Cu") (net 17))
 (segment (start 186.0218 54.0082) (end 186.0218 42.0038) (width 0.2) (layer "B.Cu") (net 17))
 (segment (start 186.0218 42.0038) (end 184.404 40.386) (width 0.2) (layer "B.Cu") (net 17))
 (segment (start 166.9691 41.5275) (end 120.7598 41.5275) (width 0.2) (layer "F.Cu") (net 26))
 (segment (start 113.538 32.004) (end 113.538 34.3057) (width 0.2) (layer "F.Cu") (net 26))
 (segment (start 120.7598 41.5275) (end 113.538 34.3057) (width 0.2) (layer "F.Cu") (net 26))
 (via (at 166.9691 41.5275) (size 0.6) (drill 0.3) (layers "F.Cu" "B.Cu") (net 26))
 (segment (start 168.3676 42.926) (end 166.9691 41.5275) (width 0.2) (layer "B.Cu") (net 26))
 (segment (start 184.404 42.926) (end 168.3676 42.926) (width 0.2) (layer "B.Cu") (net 26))
 (segment (start 132.8573 76.7007) (end 123.844 76.7007) (width 0.2) (layer "F.Cu") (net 4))
 (segment (start 123.844 76.7007) (end 123.818 76.6747) (width 0.2) (layer "F.Cu") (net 4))
 (segment (start 134.3552 73.0973) (end 133.576 73.8765) (width 0.2) (layer "F.Cu") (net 4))
 (segment (start 133.576 75.982) (end 132.8573 76.7007) (width 0.2) (layer "F.Cu") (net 4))
 (segment (start 133.576 73.8765) (end 133.576 75.982) (width 0.2) (layer "F.Cu") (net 4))
 (segment (start 123.818 74.373) (end 123.818 76.6747) (width 0.2) (layer "F.Cu") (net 4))
 (segment (start 142.466 74.399) (end 142.466 73.0973) (width 0.2) (layer "F.Cu") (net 4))
 (segment (start 142.466 73.0973) (end 134.3552 73.0973) (width 0.2) (layer "F.Cu") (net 4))
 (segment (start 123.818 74.373) (end 123.818 73.0713) (width 0.2) (layer "B.Cu") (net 4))
 (segment (start 131.318 65.5713) (end 123.818 73.0713) (width 0.2) (layer "B.Cu") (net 4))
 (segment (start 131.318 57.404) (end 131.318 65.5713) (width 0.2) (layer "B.Cu") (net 4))
 (segment (start 128.778 32.004) (end 128.778 34.3057) (width 0.2) (layer "F.Cu") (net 14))
 (segment (start 173.2437 34.3057) (end 184.404 45.466) (width 0.2) (layer "F.Cu") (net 14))
 (segment (start 128.778 34.3057) (end 173.2437 34.3057) (width 0.2) (layer "F.Cu") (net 14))
 (segment (start 185.5701 51.9199) (end 185.5701 46.6321) (width 0.2) (layer "B.Cu") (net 14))
 (segment (start 184.404 53.086) (end 185.5701 51.9199) (width 0.2) (layer "B.Cu") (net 14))
 (segment (start 185.5701 46.6321) (end 184.404 45.466) (width 0.2) (layer "B.Cu") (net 14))
 (segment (start 129.1867 52.1536) (end 152.801 52.1536) (width 0.2) (layer "F.Cu") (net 30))
 (segment (start 128.778 52.5623) (end 129.1867 52.1536) (width 0.2) (layer "F.Cu") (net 30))
 (segment (start 128.778 54.864) (end 128.778 52.5623) (width 0.2) (layer "F.Cu") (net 30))
 (via (at 152.801 52.1536) (size 0.6) (drill 0.3) (layers "F.Cu" "B.Cu") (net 30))
 (segment (start 169.6486 35.306) (end 152.801 52.1536) (width 0.2) (layer "B.Cu") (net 30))
 (segment (start 184.404 35.306) (end 169.6486 35.306) (width 0.2) (layer "B.Cu") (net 30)))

